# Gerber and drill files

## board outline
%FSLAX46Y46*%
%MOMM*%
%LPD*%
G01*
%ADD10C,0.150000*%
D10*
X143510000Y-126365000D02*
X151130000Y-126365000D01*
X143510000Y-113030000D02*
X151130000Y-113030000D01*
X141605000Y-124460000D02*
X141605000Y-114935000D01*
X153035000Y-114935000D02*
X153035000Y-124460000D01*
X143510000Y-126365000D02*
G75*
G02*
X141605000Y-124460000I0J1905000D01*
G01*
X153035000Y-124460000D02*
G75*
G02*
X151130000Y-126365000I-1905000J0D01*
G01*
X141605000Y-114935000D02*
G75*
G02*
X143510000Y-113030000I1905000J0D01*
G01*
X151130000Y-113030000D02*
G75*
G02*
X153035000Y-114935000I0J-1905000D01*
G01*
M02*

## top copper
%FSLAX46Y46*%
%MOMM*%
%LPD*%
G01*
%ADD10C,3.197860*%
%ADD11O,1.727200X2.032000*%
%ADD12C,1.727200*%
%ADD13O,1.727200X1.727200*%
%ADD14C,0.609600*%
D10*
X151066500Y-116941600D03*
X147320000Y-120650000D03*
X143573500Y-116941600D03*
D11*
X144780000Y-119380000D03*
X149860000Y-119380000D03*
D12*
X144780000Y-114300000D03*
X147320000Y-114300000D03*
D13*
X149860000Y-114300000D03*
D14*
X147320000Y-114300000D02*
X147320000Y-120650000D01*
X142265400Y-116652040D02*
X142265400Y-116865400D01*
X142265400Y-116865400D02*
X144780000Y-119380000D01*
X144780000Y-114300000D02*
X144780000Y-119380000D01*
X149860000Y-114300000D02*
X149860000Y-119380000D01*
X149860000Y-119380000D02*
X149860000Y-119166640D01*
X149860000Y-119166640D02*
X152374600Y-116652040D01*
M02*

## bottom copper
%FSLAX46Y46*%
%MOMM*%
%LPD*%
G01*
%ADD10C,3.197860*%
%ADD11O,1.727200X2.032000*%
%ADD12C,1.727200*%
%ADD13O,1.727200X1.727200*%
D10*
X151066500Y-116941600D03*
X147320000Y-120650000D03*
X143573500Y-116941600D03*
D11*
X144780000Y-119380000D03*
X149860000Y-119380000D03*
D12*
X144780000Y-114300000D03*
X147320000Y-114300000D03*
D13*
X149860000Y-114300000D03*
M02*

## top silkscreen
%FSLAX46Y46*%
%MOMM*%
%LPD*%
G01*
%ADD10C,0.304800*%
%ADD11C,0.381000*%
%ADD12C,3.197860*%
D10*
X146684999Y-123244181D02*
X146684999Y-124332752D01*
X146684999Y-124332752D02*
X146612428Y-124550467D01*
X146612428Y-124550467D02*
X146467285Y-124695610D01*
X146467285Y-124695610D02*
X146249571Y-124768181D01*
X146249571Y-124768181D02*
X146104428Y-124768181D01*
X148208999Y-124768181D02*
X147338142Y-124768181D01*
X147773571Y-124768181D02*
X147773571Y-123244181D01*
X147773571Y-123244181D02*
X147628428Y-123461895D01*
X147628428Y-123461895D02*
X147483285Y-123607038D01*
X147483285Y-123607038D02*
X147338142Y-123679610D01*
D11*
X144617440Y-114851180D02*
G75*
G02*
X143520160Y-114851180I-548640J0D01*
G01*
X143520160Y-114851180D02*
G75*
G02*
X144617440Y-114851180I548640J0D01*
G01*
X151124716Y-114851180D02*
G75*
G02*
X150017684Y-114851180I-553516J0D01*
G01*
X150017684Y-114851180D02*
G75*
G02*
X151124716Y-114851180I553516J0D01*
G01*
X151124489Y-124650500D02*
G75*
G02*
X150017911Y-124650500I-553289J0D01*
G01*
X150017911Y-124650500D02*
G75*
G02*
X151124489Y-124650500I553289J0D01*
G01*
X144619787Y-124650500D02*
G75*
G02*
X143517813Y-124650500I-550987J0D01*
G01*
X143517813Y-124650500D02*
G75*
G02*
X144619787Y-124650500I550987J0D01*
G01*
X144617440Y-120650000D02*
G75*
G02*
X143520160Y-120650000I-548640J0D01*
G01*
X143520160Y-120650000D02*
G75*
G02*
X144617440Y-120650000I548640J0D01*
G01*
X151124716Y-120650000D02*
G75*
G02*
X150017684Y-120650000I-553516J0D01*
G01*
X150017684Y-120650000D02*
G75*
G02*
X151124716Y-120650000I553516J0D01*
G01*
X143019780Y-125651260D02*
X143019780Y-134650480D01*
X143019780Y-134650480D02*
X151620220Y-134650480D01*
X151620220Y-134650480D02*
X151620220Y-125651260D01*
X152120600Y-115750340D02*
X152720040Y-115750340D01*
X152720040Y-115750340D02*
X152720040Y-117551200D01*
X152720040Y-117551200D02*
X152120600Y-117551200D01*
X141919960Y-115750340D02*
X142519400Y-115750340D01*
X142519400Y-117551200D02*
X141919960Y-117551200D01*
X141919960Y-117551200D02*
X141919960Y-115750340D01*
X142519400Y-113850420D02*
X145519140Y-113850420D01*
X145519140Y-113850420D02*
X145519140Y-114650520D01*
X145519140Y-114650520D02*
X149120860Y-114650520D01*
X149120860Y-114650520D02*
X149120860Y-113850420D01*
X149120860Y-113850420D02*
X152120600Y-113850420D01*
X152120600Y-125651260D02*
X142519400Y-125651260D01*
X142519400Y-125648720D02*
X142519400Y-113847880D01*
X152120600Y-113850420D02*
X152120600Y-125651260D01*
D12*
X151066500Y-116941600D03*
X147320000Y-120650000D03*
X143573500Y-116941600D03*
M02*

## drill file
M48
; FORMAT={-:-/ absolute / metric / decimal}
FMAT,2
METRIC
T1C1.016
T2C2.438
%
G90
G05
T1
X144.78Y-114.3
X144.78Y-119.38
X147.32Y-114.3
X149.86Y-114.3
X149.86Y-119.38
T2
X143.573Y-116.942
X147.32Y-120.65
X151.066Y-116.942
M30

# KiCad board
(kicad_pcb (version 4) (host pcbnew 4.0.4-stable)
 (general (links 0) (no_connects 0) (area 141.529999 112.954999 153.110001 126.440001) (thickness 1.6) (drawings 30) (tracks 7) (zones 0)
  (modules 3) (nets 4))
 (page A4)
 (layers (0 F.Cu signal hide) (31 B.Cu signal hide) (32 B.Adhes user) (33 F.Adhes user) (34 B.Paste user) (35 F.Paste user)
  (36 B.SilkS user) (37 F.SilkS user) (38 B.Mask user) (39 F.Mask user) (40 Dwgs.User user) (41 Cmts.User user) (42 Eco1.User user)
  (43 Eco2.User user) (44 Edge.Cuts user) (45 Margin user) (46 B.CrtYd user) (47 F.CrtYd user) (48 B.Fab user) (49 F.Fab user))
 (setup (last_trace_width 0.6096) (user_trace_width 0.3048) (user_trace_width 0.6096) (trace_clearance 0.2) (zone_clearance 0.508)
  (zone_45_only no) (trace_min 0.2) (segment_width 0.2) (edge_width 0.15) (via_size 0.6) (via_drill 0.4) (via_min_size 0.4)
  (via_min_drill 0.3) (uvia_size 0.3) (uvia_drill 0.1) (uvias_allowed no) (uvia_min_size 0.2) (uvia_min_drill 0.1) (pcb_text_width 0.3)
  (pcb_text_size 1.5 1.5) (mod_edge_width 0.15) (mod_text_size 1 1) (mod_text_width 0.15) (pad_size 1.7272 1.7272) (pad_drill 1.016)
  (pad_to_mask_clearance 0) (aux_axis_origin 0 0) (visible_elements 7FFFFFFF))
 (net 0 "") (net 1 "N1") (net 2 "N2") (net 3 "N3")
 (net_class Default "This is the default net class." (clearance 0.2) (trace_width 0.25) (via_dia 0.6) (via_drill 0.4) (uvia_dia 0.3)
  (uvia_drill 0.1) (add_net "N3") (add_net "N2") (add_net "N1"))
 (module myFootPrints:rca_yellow (layer F.Cu) (at 147.32 120.65)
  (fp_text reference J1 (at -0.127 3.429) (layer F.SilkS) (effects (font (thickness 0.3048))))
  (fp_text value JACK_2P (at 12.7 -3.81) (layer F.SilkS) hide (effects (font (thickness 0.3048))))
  (fp_circle (center -3.2512 -5.79882) (end -3.79984 -5.79882) (layer F.SilkS) (width 0.381))
  (fp_circle (center 3.2512 -5.79882) (end 2.70002 -5.84962) (layer F.SilkS) (width 0.381))
  (fp_circle (center 3.2512 4.0005) (end 2.70002 4.04876) (layer F.SilkS) (width 0.381))
  (fp_circle (center -3.2512 4.0005) (end -3.79984 3.9497) (layer F.SilkS) (width 0.381))
  (fp_circle (center -3.2512 0) (end -3.79984 0) (layer F.SilkS) (width 0.381))
  (fp_circle (center 3.2512 0) (end 2.70002 -0.0508) (layer F.SilkS) (width 0.381))
  (fp_line (start -4.30022 5.00126) (end -4.30022 14.00048) (layer F.SilkS) (width 0.381))
  (fp_line (start -4.30022 14.00048) (end 4.30022 14.00048) (layer F.SilkS) (width 0.381))
  (fp_line (start 4.30022 14.00048) (end 4.30022 5.00126) (layer F.SilkS) (width 0.381))
  (fp_line (start 4.8006 -4.89966) (end 5.40004 -4.89966) (layer F.SilkS) (width 0.381))
  (fp_line (start 5.40004 -4.89966) (end 5.40004 -3.0988) (layer F.SilkS) (width 0.381))
  (fp_line (start 5.40004 -3.0988) (end 4.8006 -3.0988) (layer F.SilkS) (width 0.381))
  (fp_line (start -5.40004 -4.89966) (end -4.8006 -4.89966) (layer F.SilkS) (width 0.381))
  (fp_line (start -4.8006 -3.0988) (end -5.40004 -3.0988) (layer F.SilkS) (width 0.381))
  (fp_line (start -5.40004 -3.0988) (end -5.40004 -4.89966) (layer F.SilkS) (width 0.381))
  (fp_line (start -4.8006 -6.79958) (end -1.80086 -6.79958) (layer F.SilkS) (width 0.381))
  (fp_line (start -1.80086 -6.79958) (end -1.80086 -5.99948) (layer F.SilkS) (width 0.381))
  (fp_line (start -1.80086 -5.99948) (end 1.80086 -5.99948) (layer F.SilkS) (width 0.381))
  (fp_line (start 1.80086 -5.99948) (end 1.80086 -6.79958) (layer F.SilkS) (width 0.381))
  (fp_line (start 1.80086 -6.79958) (end 4.8006 -6.79958) (layer F.SilkS) (width 0.381))
  (fp_line (start 4.8006 5.00126) (end -4.8006 5.00126) (layer F.SilkS) (width 0.381))
  (fp_line (start -4.8006 4.99872) (end -4.8006 -6.80212) (layer F.SilkS) (width 0.381))
  (fp_line (start 4.8006 -6.79958) (end 4.8006 5.00126) (layer F.SilkS) (width 0.381))
  (pad 3 thru_hole circle (at 3.7465 -3.7084) (size 3.19786 3.19786) (drill 2.4384) (layers *.Cu *.Mask F.SilkS) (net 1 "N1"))
  (pad 2 thru_hole circle (at 0 0) (size 3.19786 3.19786) (drill 2.4384) (layers *.Cu *.Mask F.SilkS) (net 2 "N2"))
  (pad 1 thru_hole circle (at -3.7465 -3.7084) (size 3.19786 3.19786) (drill 2.4384) (layers *.Cu *.Mask F.SilkS) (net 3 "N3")))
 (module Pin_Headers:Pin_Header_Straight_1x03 (layer B.Cu) (at 144.78 119.38 270)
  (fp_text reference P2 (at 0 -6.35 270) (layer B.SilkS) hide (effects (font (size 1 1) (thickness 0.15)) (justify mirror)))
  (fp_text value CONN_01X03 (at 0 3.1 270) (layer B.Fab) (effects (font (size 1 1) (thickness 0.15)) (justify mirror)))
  (pad 1 thru_hole oval (at 0 0 270) (size 2.032 1.7272) (drill 1.016) (layers *.Cu *.Mask B.SilkS) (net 3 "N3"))
  (pad 3 thru_hole oval (at 0 -5.08 270) (size 2.032 1.7272) (drill 1.016) (layers *.Cu *.Mask B.SilkS) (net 1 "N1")))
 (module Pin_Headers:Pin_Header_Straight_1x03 (layer B.Cu) (at 144.78 114.3 270)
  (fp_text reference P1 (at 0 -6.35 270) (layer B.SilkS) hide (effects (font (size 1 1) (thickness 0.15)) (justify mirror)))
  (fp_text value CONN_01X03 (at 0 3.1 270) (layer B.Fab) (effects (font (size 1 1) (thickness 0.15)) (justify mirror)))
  (pad 1 thru_hole circle (at 0 0 270) (size 1.7272 1.7272) (drill 1.016) (layers *.Cu *.Mask B.SilkS) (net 3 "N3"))
  (pad 2 thru_hole circle (at 0 -2.54 270) (size 1.7272 1.7272) (drill 1.016) (layers *.Cu *.Mask B.SilkS) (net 2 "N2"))
  (pad 3 thru_hole oval (at 0 -5.08 270) (size 1.7272 1.7272) (drill 1.016) (layers *.Cu *.Mask B.SilkS) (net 1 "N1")))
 (gr_line (start 143.51 126.365) (end 151.13 126.365) (angle 90) (layer Edge.Cuts) (width 0.15))
 (gr_line (start 143.51 113.03) (end 151.13 113.03) (angle 90) (layer Edge.Cuts) (width 0.15))
 (gr_line (start 141.605 124.46) (end 141.605 114.935) (angle 90) (layer Edge.Cuts) (width 0.15))
 (gr_line (start 153.035 114.935) (end 153.035 124.46) (angle 90) (layer Edge.Cuts) (width 0.15))
 (gr_arc (start 143.51 124.46) (end 143.51 126.365) (angle 90) (layer Edge.Cuts) (width 0.15))
 (gr_arc (start 151.13 124.46) (end 153.035 124.46) (angle 90) (layer Edge.Cuts) (width 0.15))
 (gr_arc (start 143.51 114.935) (end 141.605 114.935) (angle 90) (layer Edge.Cuts) (width 0.15))
 (gr_arc (start 151.13 114.935) (end 151.13 113.03) (angle 90) (layer Edge.Cuts) (width 0.15))
 (segment (start 147.32 114.3) (end 147.32 120.65) (width 0.6096) (layer F.Cu) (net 2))
 (segment (start 142.2654 116.65204) (end 142.2654 116.8654) (width 0.6096) (layer F.Cu) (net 3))
 (segment (start 142.2654 116.8654) (end 144.78 119.38) (width 0.6096) (layer F.Cu) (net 3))
 (segment (start 144.78 114.3) (end 144.78 119.38) (width 0.6096) (layer F.Cu) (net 3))
 (segment (start 149.86 114.3) (end 149.86 119.38) (width 0.6096) (layer F.Cu) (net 1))
 (segment (start 149.86 119.38) (end 149.86 119.16664) (width 0.6096) (layer F.Cu) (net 1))
 (segment (start 149.86 119.16664) (end 152.3746 116.65204) (width 0.6096) (layer F.Cu) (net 1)))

